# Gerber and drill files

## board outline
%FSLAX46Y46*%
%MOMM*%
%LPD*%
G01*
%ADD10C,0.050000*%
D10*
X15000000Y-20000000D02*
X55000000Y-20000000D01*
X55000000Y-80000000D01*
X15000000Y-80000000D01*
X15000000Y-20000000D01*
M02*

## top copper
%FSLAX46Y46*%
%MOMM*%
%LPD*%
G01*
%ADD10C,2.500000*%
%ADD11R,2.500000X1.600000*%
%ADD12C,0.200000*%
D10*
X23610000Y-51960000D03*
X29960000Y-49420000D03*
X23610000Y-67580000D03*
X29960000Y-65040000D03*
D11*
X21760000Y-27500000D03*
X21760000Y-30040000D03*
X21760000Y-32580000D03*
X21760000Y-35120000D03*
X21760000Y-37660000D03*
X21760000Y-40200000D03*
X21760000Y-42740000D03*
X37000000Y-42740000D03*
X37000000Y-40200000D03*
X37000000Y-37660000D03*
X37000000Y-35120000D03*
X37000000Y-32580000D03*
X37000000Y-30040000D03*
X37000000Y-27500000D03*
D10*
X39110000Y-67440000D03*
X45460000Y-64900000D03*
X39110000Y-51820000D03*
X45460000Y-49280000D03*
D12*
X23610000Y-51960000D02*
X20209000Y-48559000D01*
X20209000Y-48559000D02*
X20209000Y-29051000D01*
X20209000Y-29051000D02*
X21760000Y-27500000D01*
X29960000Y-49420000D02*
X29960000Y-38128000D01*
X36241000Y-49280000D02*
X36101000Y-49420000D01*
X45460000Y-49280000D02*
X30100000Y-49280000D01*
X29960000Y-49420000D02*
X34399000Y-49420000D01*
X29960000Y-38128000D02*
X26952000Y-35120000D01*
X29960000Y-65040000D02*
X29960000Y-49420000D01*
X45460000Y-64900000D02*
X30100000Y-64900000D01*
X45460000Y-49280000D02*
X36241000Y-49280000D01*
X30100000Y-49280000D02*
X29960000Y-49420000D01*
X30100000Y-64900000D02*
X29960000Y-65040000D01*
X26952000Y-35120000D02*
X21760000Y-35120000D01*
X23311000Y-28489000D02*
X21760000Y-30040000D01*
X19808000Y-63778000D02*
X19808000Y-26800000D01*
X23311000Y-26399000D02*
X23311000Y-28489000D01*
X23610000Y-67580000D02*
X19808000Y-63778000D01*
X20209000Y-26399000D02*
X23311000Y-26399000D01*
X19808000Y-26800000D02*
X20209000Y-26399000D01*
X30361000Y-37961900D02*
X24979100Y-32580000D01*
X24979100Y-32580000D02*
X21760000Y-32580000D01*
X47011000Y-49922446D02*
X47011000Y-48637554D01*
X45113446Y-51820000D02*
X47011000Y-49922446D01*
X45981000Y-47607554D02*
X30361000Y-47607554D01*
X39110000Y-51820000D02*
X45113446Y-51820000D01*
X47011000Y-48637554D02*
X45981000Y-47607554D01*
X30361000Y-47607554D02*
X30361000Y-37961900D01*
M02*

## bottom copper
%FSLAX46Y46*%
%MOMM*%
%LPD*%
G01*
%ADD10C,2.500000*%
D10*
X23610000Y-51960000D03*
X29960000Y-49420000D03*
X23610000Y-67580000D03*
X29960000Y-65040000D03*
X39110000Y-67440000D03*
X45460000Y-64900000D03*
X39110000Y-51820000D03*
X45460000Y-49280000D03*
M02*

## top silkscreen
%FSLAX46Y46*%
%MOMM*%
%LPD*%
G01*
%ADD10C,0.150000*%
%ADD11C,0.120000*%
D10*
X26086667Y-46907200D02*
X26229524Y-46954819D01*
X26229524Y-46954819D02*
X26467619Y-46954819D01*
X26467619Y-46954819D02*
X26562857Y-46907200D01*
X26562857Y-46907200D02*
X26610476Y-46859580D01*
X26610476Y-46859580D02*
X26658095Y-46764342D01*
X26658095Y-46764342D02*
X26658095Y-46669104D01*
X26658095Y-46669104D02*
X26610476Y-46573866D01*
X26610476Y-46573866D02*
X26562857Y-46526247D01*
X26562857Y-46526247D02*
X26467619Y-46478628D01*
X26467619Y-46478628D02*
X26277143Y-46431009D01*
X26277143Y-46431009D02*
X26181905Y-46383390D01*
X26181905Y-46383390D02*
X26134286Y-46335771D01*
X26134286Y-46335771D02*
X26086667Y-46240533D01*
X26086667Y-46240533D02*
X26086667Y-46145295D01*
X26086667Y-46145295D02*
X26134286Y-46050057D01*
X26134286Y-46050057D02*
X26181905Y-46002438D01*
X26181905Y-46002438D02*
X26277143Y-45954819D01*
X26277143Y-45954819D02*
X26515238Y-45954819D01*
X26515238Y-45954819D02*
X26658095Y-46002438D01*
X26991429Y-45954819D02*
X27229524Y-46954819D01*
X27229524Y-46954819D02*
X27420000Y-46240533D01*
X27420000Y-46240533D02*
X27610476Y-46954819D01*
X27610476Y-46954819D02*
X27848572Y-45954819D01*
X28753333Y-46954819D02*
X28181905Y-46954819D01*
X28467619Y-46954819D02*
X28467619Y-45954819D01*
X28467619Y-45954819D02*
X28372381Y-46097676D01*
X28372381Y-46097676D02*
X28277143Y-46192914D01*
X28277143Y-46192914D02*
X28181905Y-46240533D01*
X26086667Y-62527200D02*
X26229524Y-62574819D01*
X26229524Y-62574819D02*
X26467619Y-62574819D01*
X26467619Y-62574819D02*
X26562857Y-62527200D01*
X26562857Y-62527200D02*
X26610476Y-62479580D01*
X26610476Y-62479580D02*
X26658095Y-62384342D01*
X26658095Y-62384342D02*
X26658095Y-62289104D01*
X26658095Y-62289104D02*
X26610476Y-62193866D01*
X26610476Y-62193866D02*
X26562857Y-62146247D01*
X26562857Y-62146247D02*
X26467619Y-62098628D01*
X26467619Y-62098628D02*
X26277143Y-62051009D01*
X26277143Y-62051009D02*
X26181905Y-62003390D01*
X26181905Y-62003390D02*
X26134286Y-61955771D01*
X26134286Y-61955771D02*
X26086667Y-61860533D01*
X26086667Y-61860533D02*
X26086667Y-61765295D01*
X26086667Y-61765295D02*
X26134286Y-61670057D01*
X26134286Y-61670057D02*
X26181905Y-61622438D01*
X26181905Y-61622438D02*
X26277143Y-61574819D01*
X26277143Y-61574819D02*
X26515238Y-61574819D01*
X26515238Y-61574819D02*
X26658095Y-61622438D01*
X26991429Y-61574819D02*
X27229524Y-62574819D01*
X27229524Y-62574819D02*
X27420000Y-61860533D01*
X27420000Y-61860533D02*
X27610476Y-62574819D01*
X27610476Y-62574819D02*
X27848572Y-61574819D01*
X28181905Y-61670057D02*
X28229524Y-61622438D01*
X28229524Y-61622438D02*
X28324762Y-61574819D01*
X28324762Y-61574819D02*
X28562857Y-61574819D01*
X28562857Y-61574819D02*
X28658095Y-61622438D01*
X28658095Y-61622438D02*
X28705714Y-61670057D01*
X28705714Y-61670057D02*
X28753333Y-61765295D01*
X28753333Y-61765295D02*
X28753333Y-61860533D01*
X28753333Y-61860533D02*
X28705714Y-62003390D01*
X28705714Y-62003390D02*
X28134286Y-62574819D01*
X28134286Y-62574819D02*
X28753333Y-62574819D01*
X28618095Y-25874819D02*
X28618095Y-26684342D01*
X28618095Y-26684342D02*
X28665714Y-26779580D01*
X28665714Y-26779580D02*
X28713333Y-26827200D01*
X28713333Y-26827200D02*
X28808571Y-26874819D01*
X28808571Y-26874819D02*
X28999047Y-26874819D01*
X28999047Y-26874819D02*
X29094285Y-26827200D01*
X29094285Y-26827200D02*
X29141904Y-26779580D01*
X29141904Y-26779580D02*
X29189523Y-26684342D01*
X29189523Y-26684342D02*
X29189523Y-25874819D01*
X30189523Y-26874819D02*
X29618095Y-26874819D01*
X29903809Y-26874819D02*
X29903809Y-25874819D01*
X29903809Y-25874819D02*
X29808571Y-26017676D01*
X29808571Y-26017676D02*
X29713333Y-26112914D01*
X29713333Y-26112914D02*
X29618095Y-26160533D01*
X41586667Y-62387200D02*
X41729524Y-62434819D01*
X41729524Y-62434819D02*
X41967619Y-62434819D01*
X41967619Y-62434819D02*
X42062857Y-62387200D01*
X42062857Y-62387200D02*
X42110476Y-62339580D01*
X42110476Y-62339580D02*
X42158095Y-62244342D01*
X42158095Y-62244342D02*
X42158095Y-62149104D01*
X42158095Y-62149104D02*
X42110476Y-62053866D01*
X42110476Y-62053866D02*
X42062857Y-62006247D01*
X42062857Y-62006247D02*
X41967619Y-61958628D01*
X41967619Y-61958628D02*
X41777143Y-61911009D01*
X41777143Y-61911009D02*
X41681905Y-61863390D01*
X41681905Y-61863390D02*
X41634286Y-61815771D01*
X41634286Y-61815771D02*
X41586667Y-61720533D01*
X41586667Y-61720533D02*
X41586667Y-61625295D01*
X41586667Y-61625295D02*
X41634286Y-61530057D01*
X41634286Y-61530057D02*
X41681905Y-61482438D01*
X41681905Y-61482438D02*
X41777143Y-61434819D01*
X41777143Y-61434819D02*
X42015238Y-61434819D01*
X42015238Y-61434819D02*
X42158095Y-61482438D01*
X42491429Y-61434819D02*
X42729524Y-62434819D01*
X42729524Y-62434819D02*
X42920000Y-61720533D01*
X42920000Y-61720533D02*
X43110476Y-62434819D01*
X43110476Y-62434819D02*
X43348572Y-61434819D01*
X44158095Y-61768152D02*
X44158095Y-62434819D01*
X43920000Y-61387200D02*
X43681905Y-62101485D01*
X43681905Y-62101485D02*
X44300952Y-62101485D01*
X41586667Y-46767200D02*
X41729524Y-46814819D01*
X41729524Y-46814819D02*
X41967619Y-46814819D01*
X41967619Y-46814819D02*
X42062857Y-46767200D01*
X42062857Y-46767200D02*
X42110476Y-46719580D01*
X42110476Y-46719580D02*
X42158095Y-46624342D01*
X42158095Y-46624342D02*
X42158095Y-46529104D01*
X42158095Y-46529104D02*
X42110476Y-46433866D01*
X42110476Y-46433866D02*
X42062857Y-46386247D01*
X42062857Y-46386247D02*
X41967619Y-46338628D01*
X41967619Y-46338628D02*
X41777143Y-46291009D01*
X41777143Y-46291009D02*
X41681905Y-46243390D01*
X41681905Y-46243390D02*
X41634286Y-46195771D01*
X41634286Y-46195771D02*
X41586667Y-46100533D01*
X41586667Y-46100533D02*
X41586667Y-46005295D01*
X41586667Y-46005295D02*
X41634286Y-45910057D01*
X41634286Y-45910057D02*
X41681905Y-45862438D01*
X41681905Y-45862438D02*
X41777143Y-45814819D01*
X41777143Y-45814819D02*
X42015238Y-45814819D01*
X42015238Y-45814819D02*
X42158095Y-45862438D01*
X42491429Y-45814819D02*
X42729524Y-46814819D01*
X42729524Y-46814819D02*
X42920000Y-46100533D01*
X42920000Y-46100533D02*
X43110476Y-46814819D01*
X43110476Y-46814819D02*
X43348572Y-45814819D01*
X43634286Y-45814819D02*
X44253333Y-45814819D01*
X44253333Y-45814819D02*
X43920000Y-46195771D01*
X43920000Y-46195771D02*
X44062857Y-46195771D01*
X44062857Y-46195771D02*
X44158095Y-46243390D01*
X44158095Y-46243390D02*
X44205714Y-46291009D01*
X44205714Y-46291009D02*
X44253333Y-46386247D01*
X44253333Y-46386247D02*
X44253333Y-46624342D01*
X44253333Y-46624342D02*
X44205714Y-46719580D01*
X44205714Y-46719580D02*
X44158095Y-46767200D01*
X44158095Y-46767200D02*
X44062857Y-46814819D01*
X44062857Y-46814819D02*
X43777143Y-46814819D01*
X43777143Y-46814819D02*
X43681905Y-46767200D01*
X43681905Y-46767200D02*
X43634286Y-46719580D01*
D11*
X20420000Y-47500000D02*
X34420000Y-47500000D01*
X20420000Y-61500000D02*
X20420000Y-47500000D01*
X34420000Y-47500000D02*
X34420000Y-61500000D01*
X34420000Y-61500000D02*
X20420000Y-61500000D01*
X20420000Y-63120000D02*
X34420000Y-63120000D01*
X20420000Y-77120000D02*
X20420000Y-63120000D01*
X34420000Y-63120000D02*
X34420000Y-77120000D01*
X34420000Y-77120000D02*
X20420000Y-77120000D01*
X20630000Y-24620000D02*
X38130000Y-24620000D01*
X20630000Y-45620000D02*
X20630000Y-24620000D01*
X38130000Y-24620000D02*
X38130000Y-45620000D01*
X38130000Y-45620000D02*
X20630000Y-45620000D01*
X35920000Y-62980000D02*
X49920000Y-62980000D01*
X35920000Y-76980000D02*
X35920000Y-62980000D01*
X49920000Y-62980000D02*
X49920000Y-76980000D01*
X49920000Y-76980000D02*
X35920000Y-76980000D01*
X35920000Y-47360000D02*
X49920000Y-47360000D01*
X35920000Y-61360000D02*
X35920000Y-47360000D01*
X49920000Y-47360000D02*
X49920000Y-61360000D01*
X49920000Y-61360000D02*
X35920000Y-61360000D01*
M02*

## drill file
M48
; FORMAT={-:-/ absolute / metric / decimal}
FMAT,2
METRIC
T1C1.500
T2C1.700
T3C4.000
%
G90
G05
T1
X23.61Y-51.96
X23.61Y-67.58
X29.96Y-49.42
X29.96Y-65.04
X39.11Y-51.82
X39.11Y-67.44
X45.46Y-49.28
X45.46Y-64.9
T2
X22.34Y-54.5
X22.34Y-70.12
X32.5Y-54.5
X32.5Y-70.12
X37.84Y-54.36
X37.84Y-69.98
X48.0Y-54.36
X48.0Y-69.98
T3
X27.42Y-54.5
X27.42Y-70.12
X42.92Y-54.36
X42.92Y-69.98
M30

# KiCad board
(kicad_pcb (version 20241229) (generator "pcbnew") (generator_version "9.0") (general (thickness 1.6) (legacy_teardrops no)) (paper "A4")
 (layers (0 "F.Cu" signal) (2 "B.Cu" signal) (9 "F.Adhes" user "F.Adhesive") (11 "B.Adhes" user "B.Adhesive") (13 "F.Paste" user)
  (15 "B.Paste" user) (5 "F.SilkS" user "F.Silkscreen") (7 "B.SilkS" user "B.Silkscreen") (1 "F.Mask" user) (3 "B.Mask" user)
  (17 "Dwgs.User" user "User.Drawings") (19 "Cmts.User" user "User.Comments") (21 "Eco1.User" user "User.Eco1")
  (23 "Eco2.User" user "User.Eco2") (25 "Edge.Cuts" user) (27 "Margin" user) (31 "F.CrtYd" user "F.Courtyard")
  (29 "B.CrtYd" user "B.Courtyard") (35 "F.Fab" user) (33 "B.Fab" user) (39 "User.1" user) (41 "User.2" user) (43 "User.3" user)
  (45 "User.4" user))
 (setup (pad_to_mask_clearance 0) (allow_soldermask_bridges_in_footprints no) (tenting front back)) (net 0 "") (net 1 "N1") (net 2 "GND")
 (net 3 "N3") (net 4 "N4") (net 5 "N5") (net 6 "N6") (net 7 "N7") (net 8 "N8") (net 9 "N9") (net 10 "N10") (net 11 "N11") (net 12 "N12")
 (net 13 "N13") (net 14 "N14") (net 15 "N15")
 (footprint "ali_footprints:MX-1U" (layer "F.Cu") (at 27.42 54.5)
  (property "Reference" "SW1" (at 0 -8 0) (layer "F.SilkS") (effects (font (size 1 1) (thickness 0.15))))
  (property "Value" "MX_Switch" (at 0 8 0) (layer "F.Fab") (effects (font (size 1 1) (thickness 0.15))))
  (fp_line (start -7 -7) (end 7 -7) (stroke (width 0.12) (type solid)) (layer "F.SilkS"))
  (fp_line (start -7 7) (end -7 -7) (stroke (width 0.12) (type solid)) (layer "F.SilkS"))
  (fp_line (start 7 -7) (end 7 7) (stroke (width 0.12) (type solid)) (layer "F.SilkS"))
  (fp_line (start 7 7) (end -7 7) (stroke (width 0.12) (type solid)) (layer "F.SilkS"))
  (pad "" np_thru_hole circle (at -5.08 0) (size 1.7 1.7) (drill 1.7) (layers "*.Cu" "*.Mask"))
  (pad "" np_thru_hole circle (at 0 0) (size 4 4) (drill 4) (layers "*.Cu" "*.Mask"))
  (pad "" np_thru_hole circle (at 5.08 0) (size 1.7 1.7) (drill 1.7) (layers "*.Cu" "*.Mask"))
  (pad "1" thru_hole circle (at -3.81 -2.54) (size 2.5 2.5) (drill 1.5) (layers "*.Cu" "*.Mask") (remove_unused_layers no) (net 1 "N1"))
  (pad "2" thru_hole circle (at 2.54 -5.08) (size 2.5 2.5) (drill 1.5) (layers "*.Cu" "*.Mask") (remove_unused_layers no) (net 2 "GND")))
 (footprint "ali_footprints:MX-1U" (layer "F.Cu") (at 27.42 70.12)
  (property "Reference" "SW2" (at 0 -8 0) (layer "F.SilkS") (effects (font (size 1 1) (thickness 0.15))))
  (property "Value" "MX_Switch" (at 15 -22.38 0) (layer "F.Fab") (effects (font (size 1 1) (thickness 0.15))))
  (fp_line (start -7 -7) (end 7 -7) (stroke (width 0.12) (type solid)) (layer "F.SilkS"))
  (fp_line (start -7 7) (end -7 -7) (stroke (width 0.12) (type solid)) (layer "F.SilkS"))
  (fp_line (start 7 -7) (end 7 7) (stroke (width 0.12) (type solid)) (layer "F.SilkS"))
  (fp_line (start 7 7) (end -7 7) (stroke (width 0.12) (type solid)) (layer "F.SilkS"))
  (pad "" np_thru_hole circle (at -5.08 0) (size 1.7 1.7) (drill 1.7) (layers "*.Cu" "*.Mask"))
  (pad "" np_thru_hole circle (at 0 0) (size 4 4) (drill 4) (layers "*.Cu" "*.Mask"))
  (pad "" np_thru_hole circle (at 5.08 0) (size 1.7 1.7) (drill 1.7) (layers "*.Cu" "*.Mask"))
  (pad "1" thru_hole circle (at -3.81 -2.54) (size 2.5 2.5) (drill 1.5) (layers "*.Cu" "*.Mask") (remove_unused_layers no) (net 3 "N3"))
  (pad "2" thru_hole circle (at 2.54 -5.08) (size 2.5 2.5) (drill 1.5) (layers "*.Cu" "*.Mask") (remove_unused_layers no) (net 2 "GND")))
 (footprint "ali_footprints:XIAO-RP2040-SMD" (layer "F.Cu") (at 29.38 35.12)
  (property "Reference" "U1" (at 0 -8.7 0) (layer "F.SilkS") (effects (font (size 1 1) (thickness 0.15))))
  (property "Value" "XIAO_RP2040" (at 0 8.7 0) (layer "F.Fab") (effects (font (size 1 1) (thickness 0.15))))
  (fp_line (start -8.75 -10.5) (end 8.75 -10.5) (stroke (width 0.12) (type solid)) (layer "F.SilkS"))
  (fp_line (start -8.75 10.5) (end -8.75 -10.5) (stroke (width 0.12) (type solid)) (layer "F.SilkS"))
  (fp_line (start 8.75 -10.5) (end 8.75 10.5) (stroke (width 0.12) (type solid)) (layer "F.SilkS"))
  (fp_line (start 8.75 10.5) (end -8.75 10.5) (stroke (width 0.12) (type solid)) (layer "F.SilkS"))
  (pad "1" smd rect (at -7.62 -7.62) (size 2.5 1.6) (layers "F.Cu" "F.Mask" "F.Paste") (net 1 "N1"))
  (pad "2" smd rect (at -7.62 -5.08) (size 2.5 1.6) (layers "F.Cu" "F.Mask" "F.Paste") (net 3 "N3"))
  (pad "3" smd rect (at -7.62 -2.54) (size 2.5 1.6) (layers "F.Cu" "F.Mask" "F.Paste") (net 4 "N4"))
  (pad "4" smd rect (at -7.62 0) (size 2.5 1.6) (layers "F.Cu" "F.Mask" "F.Paste") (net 2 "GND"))
  (pad "5" smd rect (at -7.62 2.54) (size 2.5 1.6) (layers "F.Cu" "F.Mask" "F.Paste") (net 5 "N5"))
  (pad "6" smd rect (at -7.62 5.08) (size 2.5 1.6) (layers "F.Cu" "F.Mask" "F.Paste") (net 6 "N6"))
  (pad "7" smd rect (at -7.62 7.62) (size 2.5 1.6) (layers "F.Cu" "F.Mask" "F.Paste") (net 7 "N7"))
  (pad "8" smd rect (at 7.62 7.62) (size 2.5 1.6) (layers "F.Cu" "F.Mask" "F.Paste") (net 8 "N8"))
  (pad "9" smd rect (at 7.62 5.08) (size 2.5 1.6) (layers "F.Cu" "F.Mask" "F.Paste") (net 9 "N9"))
  (pad "10" smd rect (at 7.62 2.54) (size 2.5 1.6) (layers "F.Cu" "F.Mask" "F.Paste") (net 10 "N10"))
  (pad "11" smd rect (at 7.62 0) (size 2.5 1.6) (layers "F.Cu" "F.Mask" "F.Paste") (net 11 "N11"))
  (pad "12" smd rect (at 7.62 -2.54) (size 2.5 1.6) (layers "F.Cu" "F.Mask" "F.Paste") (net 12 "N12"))
  (pad "13" smd rect (at 7.62 -5.08) (size 2.5 1.6) (layers "F.Cu" "F.Mask" "F.Paste") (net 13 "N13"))
  (pad "14" smd rect (at 7.62 -7.62) (size 2.5 1.6) (layers "F.Cu" "F.Mask" "F.Paste") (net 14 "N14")))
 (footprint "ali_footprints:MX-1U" (layer "F.Cu") (at 42.92 69.98)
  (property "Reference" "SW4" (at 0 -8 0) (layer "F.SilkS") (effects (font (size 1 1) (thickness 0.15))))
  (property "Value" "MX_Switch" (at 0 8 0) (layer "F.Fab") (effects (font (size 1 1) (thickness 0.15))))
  (fp_line (start -7 -7) (end 7 -7) (stroke (width 0.12) (type solid)) (layer "F.SilkS"))
  (fp_line (start -7 7) (end -7 -7) (stroke (width 0.12) (type solid)) (layer "F.SilkS"))
  (fp_line (start 7 -7) (end 7 7) (stroke (width 0.12) (type solid)) (layer "F.SilkS"))
  (fp_line (start 7 7) (end -7 7) (stroke (width 0.12) (type solid)) (layer "F.SilkS"))
  (pad "" np_thru_hole circle (at -5.08 0) (size 1.7 1.7) (drill 1.7) (layers "*.Cu" "*.Mask"))
  (pad "" np_thru_hole circle (at 0 0) (size 4 4) (drill 4) (layers "*.Cu" "*.Mask"))
  (pad "" np_thru_hole circle (at 5.08 0) (size 1.7 1.7) (drill 1.7) (layers "*.Cu" "*.Mask"))
  (pad "1" thru_hole circle (at -3.81 -2.54) (size 2.5 2.5) (drill 1.5) (layers "*.Cu" "*.Mask") (remove_unused_layers no) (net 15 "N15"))
  (pad "2" thru_hole circle (at 2.54 -5.08) (size 2.5 2.5) (drill 1.5) (layers "*.Cu" "*.Mask") (remove_unused_layers no) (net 2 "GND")))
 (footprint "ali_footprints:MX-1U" (layer "F.Cu") (at 42.92 54.36)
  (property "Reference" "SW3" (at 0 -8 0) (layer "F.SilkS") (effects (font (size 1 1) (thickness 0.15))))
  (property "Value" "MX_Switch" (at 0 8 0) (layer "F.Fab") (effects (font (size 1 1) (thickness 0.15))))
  (fp_line (start -7 -7) (end 7 -7) (stroke (width 0.12) (type solid)) (layer "F.SilkS"))
  (fp_line (start -7 7) (end -7 -7) (stroke (width 0.12) (type solid)) (layer "F.SilkS"))
  (fp_line (start 7 -7) (end 7 7) (stroke (width 0.12) (type solid)) (layer "F.SilkS"))
  (fp_line (start 7 7) (end -7 7) (stroke (width 0.12) (type solid)) (layer "F.SilkS"))
  (pad "" np_thru_hole circle (at -5.08 0) (size 1.7 1.7) (drill 1.7) (layers "*.Cu" "*.Mask"))
  (pad "" np_thru_hole circle (at 0 0) (size 4 4) (drill 4) (layers "*.Cu" "*.Mask"))
  (pad "" np_thru_hole circle (at 5.08 0) (size 1.7 1.7) (drill 1.7) (layers "*.Cu" "*.Mask"))
  (pad "1" thru_hole circle (at -3.81 -2.54) (size 2.5 2.5) (drill 1.5) (layers "*.Cu" "*.Mask") (remove_unused_layers no) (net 4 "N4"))
  (pad "2" thru_hole circle (at 2.54 -5.08) (size 2.5 2.5) (drill 1.5) (layers "*.Cu" "*.Mask") (remove_unused_layers no) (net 2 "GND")))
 (gr_rect (start 15 20) (end 55 80) (stroke (width 0.05) (type default)) (fill no) (layer "Edge.Cuts"))
 (segment (start 23.61 51.96) (end 20.209 48.559) (width 0.2) (layer "F.Cu") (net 1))
 (segment (start 20.209 48.559) (end 20.209 29.051) (width 0.2) (layer "F.Cu") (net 1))
 (segment (start 20.209 29.051) (end 21.76 27.5) (width 0.2) (layer "F.Cu") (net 1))
 (segment (start 29.96 49.42) (end 29.96 38.128) (width 0.2) (layer "F.Cu") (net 2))
 (segment (start 36.241 49.28) (end 36.101 49.42) (width 0.2) (layer "F.Cu") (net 2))
 (segment (start 45.46 49.28) (end 30.1 49.28) (width 0.2) (layer "F.Cu") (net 2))
 (segment (start 29.96 49.42) (end 34.399 49.42) (width 0.2) (layer "F.Cu") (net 2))
 (segment (start 29.96 38.128) (end 26.952 35.12) (width 0.2) (layer "F.Cu") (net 2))
 (segment (start 29.96 65.04) (end 29.96 49.42) (width 0.2) (layer "F.Cu") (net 2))
 (segment (start 45.46 64.9) (end 30.1 64.9) (width 0.2) (layer "F.Cu") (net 2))
 (segment (start 45.46 49.28) (end 36.241 49.28) (width 0.2) (layer "F.Cu") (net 2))
 (segment (start 30.1 49.28) (end 29.96 49.42) (width 0.2) (layer "F.Cu") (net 2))
 (segment (start 30.1 64.9) (end 29.96 65.04) (width 0.2) (layer "F.Cu") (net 2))
 (segment (start 26.952 35.12) (end 21.76 35.12) (width 0.2) (layer "F.Cu") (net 2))
 (segment (start 23.311 28.489) (end 21.76 30.04) (width 0.2) (layer "F.Cu") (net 3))
 (segment (start 19.808 63.778) (end 19.808 26.8) (width 0.2) (layer "F.Cu") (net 3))
 (segment (start 23.311 26.399) (end 23.311 28.489) (width 0.2) (layer "F.Cu") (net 3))
 (segment (start 23.61 67.58) (end 19.808 63.778) (width 0.2) (layer "F.Cu") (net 3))
 (segment (start 20.209 26.399) (end 23.311 26.399) (width 0.2) (layer "F.Cu") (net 3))
 (segment (start 19.808 26.8) (end 20.209 26.399) (width 0.2) (layer "F.Cu") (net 3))
 (segment (start 30.361 37.9619) (end 24.9791 32.58) (width 0.2) (layer "F.Cu") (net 4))
 (segment (start 24.9791 32.58) (end 21.76 32.58) (width 0.2) (layer "F.Cu") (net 4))
 (segment (start 47.011 49.922446) (end 47.011 48.637554) (width 0.2) (layer "F.Cu") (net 4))
 (segment (start 45.113446 51.82) (end 47.011 49.922446) (width 0.2) (layer "F.Cu") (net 4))
 (segment (start 45.981 47.607554) (end 30.361 47.607554) (width 0.2) (layer "F.Cu") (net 4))
 (segment (start 39.11 51.82) (end 45.113446 51.82) (width 0.2) (layer "F.Cu") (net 4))
 (segment (start 47.011 48.637554) (end 45.981 47.607554) (width 0.2) (layer "F.Cu") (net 4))
 (segment (start 30.361 47.607554) (end 30.361 37.9619) (width 0.2) (layer "F.Cu") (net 4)))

